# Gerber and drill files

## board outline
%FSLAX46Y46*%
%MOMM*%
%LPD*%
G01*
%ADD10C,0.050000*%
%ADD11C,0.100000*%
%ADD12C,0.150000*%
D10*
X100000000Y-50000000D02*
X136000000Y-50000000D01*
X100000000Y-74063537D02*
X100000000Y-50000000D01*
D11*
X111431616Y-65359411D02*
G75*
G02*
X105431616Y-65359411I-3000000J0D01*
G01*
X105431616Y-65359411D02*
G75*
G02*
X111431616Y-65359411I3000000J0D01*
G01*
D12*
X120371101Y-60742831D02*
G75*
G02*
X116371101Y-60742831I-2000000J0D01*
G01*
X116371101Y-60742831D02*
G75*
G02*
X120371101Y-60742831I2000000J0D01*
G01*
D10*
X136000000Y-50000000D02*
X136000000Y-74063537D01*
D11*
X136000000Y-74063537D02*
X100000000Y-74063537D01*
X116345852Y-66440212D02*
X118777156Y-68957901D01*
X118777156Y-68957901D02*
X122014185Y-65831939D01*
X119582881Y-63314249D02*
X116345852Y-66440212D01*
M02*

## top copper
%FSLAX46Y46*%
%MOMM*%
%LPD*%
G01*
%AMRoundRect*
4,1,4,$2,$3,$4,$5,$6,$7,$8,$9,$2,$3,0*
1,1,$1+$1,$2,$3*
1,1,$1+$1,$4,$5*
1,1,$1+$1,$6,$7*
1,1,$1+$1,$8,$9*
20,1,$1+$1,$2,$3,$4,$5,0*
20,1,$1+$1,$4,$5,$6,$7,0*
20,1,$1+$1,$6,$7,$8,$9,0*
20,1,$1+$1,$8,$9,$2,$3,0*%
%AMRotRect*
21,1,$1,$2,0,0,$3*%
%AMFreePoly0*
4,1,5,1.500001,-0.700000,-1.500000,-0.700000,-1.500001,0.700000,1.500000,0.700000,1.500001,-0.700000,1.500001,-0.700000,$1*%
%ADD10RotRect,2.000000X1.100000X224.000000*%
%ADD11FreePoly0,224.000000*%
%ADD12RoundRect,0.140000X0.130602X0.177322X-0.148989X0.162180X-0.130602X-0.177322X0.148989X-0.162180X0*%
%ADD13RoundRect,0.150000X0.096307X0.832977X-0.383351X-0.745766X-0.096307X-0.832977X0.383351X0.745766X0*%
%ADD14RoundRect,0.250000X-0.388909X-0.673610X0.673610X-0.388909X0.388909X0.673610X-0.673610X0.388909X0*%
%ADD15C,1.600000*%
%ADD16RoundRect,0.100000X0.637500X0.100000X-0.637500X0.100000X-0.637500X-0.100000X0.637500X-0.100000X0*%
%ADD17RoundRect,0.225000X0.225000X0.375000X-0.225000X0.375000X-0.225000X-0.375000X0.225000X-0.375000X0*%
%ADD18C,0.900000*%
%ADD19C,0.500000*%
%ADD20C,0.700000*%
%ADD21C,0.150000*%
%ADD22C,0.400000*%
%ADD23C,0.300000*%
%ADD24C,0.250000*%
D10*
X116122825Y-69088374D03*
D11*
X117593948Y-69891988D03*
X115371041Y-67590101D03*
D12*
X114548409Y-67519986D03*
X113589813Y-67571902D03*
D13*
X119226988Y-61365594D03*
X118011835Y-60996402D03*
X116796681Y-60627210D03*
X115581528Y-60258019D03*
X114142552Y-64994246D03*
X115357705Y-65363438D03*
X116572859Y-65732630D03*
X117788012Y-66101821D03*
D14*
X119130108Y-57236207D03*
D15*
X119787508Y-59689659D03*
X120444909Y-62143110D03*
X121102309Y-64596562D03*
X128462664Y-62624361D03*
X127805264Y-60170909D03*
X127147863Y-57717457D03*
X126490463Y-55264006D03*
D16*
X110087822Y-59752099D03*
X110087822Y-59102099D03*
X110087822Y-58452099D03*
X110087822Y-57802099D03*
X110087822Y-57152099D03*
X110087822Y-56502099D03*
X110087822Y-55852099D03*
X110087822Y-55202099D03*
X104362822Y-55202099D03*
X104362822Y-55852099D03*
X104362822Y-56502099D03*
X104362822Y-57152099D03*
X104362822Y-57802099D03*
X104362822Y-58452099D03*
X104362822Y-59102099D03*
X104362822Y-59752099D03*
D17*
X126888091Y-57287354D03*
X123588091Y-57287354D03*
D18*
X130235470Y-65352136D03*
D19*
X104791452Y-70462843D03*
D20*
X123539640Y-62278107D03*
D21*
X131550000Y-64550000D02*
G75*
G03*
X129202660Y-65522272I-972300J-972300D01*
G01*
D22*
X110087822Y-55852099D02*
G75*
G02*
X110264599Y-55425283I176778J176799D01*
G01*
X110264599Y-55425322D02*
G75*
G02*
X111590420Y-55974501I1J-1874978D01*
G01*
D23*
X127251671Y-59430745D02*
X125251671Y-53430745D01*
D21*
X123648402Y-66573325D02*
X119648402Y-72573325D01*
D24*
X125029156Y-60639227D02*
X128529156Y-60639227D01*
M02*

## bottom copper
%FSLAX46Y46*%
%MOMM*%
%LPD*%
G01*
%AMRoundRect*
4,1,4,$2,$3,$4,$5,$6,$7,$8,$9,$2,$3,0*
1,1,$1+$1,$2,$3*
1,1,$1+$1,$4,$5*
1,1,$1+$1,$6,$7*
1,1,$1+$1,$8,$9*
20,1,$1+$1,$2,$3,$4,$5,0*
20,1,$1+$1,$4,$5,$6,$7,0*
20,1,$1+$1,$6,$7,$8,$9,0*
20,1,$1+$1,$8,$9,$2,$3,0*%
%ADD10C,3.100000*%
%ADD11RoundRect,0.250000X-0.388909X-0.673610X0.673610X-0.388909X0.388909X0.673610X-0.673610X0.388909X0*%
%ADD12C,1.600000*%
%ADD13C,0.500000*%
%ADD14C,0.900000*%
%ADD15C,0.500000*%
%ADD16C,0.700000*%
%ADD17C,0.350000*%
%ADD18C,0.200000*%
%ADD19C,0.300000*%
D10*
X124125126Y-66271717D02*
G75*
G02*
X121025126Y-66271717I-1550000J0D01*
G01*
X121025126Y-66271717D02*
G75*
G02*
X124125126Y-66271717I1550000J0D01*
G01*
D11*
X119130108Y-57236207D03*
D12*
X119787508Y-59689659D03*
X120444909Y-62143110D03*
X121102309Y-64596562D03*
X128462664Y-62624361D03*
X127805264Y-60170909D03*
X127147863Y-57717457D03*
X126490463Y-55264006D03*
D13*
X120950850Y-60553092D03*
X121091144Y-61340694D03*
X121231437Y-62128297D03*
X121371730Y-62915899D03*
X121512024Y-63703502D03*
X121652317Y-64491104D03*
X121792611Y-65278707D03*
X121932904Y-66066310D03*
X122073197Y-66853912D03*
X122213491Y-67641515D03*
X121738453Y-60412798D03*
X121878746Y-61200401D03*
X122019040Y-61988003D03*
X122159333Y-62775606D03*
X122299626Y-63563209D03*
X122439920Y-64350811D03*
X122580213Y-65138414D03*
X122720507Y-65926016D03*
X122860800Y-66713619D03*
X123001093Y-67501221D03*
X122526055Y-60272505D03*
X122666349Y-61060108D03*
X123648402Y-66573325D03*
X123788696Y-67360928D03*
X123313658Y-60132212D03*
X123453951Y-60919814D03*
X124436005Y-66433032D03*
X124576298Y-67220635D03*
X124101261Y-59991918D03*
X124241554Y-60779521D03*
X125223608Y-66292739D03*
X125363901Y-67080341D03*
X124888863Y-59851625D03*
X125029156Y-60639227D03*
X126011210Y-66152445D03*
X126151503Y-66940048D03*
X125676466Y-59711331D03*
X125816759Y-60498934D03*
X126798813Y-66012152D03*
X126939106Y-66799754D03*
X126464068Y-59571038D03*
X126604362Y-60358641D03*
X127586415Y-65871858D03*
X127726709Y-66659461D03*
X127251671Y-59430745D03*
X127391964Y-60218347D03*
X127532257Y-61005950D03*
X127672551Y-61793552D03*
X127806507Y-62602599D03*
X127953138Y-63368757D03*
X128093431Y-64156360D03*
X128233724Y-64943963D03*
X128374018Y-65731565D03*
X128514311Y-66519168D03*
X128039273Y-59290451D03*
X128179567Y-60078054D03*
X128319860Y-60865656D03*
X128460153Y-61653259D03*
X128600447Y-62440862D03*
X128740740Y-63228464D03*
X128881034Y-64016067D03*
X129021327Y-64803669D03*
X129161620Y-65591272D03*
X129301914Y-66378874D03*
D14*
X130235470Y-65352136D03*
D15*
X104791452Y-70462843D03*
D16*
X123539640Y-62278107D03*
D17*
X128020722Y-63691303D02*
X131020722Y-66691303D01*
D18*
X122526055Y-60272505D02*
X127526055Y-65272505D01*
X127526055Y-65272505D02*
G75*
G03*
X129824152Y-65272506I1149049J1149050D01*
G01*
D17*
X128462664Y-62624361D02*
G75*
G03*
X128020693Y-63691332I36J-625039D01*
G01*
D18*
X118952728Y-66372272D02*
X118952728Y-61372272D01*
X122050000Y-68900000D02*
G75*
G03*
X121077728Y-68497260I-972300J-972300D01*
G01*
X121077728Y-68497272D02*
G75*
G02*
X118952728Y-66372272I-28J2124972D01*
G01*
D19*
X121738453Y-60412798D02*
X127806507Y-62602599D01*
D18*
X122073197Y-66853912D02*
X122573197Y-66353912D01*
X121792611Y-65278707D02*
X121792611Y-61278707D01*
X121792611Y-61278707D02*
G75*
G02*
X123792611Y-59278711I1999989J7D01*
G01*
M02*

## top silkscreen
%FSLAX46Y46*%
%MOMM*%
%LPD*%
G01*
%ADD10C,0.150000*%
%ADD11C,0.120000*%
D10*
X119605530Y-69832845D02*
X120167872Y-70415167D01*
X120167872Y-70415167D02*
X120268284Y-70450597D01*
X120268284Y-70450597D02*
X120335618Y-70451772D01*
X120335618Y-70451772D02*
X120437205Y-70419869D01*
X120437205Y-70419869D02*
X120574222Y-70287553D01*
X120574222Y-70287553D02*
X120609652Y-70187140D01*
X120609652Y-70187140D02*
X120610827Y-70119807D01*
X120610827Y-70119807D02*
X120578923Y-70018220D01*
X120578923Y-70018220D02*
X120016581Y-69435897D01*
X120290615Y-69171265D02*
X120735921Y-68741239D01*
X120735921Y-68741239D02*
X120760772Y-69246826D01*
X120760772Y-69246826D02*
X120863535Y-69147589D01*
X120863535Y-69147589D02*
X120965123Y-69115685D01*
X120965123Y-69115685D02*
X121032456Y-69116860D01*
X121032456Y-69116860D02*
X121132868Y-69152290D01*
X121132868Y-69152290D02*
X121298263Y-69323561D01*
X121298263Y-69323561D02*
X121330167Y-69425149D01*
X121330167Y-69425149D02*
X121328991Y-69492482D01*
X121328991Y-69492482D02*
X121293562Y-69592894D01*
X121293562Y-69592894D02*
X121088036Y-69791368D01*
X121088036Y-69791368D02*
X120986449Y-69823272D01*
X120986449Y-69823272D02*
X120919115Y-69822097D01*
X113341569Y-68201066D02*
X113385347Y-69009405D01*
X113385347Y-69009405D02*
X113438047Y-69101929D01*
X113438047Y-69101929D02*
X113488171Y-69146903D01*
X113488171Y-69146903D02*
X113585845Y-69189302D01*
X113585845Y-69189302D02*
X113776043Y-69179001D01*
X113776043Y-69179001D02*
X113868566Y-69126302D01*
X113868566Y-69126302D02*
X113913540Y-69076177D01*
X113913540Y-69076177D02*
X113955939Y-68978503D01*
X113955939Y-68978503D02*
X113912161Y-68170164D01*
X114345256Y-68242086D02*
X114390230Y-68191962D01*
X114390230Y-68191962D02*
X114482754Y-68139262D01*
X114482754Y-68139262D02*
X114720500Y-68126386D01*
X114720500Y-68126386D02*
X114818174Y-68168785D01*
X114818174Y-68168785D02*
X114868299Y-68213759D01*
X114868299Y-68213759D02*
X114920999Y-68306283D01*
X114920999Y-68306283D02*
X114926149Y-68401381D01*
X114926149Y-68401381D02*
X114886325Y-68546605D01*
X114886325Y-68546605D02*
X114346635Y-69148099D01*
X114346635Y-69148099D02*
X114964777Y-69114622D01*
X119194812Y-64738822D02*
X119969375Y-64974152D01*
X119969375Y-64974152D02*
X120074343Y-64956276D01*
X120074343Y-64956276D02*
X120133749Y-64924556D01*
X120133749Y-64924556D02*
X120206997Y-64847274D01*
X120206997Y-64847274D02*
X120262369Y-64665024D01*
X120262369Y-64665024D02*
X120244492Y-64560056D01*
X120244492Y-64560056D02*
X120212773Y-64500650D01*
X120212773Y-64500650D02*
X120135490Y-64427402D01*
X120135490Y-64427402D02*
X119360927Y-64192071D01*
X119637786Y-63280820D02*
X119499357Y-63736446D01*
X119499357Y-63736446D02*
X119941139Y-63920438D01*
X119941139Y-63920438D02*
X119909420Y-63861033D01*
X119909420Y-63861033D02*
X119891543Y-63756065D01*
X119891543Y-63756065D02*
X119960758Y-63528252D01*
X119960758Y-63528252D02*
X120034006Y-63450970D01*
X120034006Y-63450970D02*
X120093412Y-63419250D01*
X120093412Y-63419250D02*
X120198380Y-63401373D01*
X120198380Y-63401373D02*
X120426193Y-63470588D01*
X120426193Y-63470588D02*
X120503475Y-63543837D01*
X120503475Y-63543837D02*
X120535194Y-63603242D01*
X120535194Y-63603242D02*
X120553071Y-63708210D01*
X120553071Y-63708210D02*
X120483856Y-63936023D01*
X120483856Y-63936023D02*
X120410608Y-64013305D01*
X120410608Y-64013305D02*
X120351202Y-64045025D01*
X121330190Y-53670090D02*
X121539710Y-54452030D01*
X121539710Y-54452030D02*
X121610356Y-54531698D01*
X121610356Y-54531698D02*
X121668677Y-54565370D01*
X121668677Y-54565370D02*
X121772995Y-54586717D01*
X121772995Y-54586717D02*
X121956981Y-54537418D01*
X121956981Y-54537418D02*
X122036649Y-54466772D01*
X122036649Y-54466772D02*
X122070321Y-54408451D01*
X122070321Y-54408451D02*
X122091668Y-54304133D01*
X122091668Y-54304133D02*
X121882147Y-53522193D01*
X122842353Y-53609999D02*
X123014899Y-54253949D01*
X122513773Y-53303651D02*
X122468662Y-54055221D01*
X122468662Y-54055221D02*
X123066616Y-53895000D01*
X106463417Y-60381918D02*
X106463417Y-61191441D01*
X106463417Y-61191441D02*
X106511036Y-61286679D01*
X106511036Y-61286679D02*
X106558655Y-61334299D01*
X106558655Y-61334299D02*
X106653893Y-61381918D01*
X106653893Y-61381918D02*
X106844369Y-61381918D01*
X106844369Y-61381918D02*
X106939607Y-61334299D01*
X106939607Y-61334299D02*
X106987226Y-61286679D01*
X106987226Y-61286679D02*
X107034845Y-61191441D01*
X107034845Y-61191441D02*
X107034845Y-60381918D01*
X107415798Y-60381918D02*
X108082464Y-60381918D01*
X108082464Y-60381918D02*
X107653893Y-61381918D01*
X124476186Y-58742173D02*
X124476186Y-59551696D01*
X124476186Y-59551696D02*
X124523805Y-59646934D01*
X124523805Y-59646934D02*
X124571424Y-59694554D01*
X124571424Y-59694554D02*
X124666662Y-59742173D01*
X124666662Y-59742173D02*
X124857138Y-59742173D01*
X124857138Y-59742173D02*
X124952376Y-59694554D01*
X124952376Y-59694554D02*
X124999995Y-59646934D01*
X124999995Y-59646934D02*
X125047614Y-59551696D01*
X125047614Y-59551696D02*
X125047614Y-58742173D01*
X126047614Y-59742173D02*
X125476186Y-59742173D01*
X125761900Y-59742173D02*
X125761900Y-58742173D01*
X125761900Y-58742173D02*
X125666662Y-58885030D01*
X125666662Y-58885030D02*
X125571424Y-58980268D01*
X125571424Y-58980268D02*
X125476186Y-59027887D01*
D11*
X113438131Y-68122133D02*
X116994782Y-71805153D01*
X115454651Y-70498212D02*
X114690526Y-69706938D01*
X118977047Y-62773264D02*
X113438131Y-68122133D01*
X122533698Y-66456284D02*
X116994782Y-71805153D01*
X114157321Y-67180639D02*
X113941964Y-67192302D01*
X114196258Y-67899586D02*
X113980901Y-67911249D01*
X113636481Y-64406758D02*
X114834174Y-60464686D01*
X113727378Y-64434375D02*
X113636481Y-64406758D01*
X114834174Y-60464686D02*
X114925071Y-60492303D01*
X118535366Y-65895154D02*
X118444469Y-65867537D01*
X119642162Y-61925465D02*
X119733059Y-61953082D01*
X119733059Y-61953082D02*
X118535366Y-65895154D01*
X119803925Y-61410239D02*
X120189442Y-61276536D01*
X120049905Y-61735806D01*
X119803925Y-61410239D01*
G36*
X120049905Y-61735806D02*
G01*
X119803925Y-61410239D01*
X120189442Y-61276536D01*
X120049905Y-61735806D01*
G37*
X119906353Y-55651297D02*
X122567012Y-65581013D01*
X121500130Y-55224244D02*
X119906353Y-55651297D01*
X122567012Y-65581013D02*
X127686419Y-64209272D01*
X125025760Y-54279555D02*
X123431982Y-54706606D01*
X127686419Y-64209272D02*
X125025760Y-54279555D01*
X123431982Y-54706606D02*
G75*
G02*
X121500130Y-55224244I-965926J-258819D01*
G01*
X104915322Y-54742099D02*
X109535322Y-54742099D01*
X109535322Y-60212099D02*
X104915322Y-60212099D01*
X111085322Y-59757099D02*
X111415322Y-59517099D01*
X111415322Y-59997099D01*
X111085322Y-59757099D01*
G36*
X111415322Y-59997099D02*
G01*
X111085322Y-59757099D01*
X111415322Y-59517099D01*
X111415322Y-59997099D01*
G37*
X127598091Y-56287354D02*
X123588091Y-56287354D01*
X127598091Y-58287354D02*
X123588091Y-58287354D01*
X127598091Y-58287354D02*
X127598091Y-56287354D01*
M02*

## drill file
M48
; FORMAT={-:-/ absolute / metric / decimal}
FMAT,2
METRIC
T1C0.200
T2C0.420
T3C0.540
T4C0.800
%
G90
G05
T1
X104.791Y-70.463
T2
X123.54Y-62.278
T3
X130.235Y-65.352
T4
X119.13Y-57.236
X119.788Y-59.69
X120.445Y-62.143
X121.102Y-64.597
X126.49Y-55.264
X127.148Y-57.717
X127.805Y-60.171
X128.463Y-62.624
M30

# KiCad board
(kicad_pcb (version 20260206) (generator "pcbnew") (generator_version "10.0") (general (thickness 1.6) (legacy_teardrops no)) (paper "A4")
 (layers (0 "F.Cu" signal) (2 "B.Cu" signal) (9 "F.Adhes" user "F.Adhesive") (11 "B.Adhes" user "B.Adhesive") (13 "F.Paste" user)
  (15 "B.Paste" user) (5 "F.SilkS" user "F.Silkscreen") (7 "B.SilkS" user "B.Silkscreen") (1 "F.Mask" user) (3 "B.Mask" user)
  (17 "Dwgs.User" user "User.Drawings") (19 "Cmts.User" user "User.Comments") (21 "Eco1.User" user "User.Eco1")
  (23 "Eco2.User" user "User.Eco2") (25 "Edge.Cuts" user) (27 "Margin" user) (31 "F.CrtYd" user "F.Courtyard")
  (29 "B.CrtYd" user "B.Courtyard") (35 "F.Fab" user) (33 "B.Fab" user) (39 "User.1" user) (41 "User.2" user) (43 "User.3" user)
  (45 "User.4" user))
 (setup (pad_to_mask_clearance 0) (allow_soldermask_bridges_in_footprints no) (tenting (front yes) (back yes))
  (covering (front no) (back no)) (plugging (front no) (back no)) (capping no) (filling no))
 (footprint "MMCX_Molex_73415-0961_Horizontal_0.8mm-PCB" (layer "F.Cu") (at 118.101009 67.178063 -136)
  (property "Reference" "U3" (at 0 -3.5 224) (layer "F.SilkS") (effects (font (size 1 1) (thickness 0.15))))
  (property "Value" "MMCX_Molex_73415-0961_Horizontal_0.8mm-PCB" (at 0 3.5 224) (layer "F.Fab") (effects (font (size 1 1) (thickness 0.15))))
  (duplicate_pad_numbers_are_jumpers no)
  (fp_line (start 4.01 2.56) (end 4.01 -2.56) (stroke (width 0.12) (type solid)) (layer "F.SilkS"))
  (fp_line (start 4.21 -0.550001) (end 4.21 0.55) (stroke (width 0.12) (type solid)) (layer "F.SilkS"))
  (fp_line (start -3.689999 2.56) (end 4.01 2.56) (stroke (width 0.12) (type solid)) (layer "F.SilkS"))
  (fp_line (start -3.689999 -2.56) (end 4.01 -2.56) (stroke (width 0.12) (type solid)) (layer "F.SilkS"))
  (fp_line (start 0.75 1.75) (end 0.75 -1.749999) (stroke (width 0.1) (type solid)) (layer "Edge.Cuts"))
  (fp_line (start 0.75 -1.749999) (end -3.75 -1.75) (stroke (width 0.1) (type solid)) (layer "Edge.Cuts"))
  (fp_line (start -3.75 1.75) (end 0.75 1.75) (stroke (width 0.1) (type solid)) (layer "Edge.Cuts"))
  (pad "1" smd rect (at 2.75 -0.000001 224) (size 2 1.1) (layers "F.Cu" "F.Mask" "F.Paste") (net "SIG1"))
  (pad "2" smd custom (at 2.25 -1.6 224) (size 3 1.4) (layers "F.Cu" "F.Mask" "F.Paste") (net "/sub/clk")
   (options (clearance outline) (anchor rect)) (primitives))
  (pad "2" smd custom (at 2.25 1.6 224) (size 3 1.4) (layers "F.Cu" "F.Mask" "F.Paste") (options (clearance outline) (anchor rect))
   (primitives)))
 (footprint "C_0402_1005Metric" (layer "F.Cu") (at 114.069111 67.545944 -176.9)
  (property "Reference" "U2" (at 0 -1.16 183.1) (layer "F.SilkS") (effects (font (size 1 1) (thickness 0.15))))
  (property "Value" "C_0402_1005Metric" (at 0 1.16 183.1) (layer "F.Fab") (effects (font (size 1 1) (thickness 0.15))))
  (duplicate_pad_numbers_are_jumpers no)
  (fp_line (start -0.107836 0.36) (end 0.107836 0.36) (stroke (width 0.12) (type solid)) (layer "F.SilkS"))
  (fp_line (start -0.107836 -0.36) (end 0.107836 -0.36) (stroke (width 0.12) (type solid)) (layer "F.SilkS"))
  (pad "1" smd roundrect (at -0.48 0 183.1) (size 0.56 0.62) (layers "F.Cu" "F.Mask" "F.Paste") (roundrect_rratio 0.25))
  (pad "2" smd roundrect (at 0.48 0 183.1) (size 0.56 0.62) (layers "F.Cu" "F.Mask" "F.Paste") (roundrect_rratio 0.25) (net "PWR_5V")))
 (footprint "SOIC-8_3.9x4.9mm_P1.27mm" (layer "F.Cu") (at 116.68477 63.17992 -106.9)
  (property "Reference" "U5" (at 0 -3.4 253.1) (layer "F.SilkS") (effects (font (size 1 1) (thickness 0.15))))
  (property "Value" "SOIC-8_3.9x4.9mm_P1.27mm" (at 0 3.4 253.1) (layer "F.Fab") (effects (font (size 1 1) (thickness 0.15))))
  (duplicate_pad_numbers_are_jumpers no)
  (fp_line (start 2.06 2.56) (end -2.06 2.56) (stroke (width 0.12) (type solid)) (layer "F.SilkS"))
  (fp_line (start 2.06 2.465) (end 2.06 2.56) (stroke (width 0.12) (type solid)) (layer "F.SilkS"))
  (fp_line (start -2.06 2.56) (end -2.06 2.465) (stroke (width 0.12) (type solid)) (layer "F.SilkS"))
  (fp_line (start 2.06 -2.56) (end 2.06 -2.465) (stroke (width 0.12) (type solid)) (layer "F.SilkS"))
  (fp_line (start -2.06 -2.465) (end -2.06 -2.56) (stroke (width 0.12) (type solid)) (layer "F.SilkS"))
  (fp_line (start -2.06 -2.56) (end 2.06 -2.56) (stroke (width 0.12) (type solid)) (layer "F.SilkS"))
  (fp_poly (pts (xy -2.6 -2.47) (xy -2.84 -2.8) (xy -2.36 -2.8)) (stroke (width 0.12) (type solid)) (fill yes) (layer "F.SilkS"))
  (pad "1" smd roundrect (at -2.475 -1.905 253.1) (size 1.95 0.6) (layers "F.Cu" "F.Mask" "F.Paste") (roundrect_rratio 0.25) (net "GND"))
  (pad "2" smd roundrect (at -2.475 -0.635 253.1) (size 1.95 0.6) (layers "F.Cu" "F.Mask" "F.Paste") (roundrect_rratio 0.25) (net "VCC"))
  (pad "3" smd roundrect (at -2.475 0.635 253.1) (size 1.95 0.6) (layers "F.Cu" "F.Mask" "F.Paste") (roundrect_rratio 0.25))
  (pad "4" smd roundrect (at -2.475 1.905 253.1) (size 1.95 0.6) (layers "F.Cu" "F.Mask" "F.Paste") (roundrect_rratio 0.25) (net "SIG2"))
  (pad "5" smd roundrect (at 2.475 1.905 253.1) (size 1.95 0.6) (layers "F.Cu" "F.Mask" "F.Paste") (roundrect_rratio 0.25) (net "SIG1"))
  (pad "6" smd roundrect (at 2.475 0.635 253.1) (size 1.95 0.6) (layers "F.Cu" "F.Mask" "F.Paste") (roundrect_rratio 0.25))
  (pad "7" smd roundrect (at 2.475 -0.635 253.1) (size 1.95 0.6) (layers "F.Cu" "F.Mask" "F.Paste") (roundrect_rratio 0.25) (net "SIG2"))
  (pad "8" smd roundrect (at 2.475 -1.905 253.1) (size 1.95 0.6) (layers "F.Cu" "F.Mask" "F.Paste") (roundrect_rratio 0.25) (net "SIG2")))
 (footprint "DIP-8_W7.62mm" (layer "F.Cu") (at 119.130108 57.236207 15)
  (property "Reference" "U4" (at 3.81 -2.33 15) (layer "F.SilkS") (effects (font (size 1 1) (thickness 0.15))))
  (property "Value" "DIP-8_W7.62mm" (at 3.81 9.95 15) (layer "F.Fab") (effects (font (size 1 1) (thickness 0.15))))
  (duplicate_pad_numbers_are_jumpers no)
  (fp_line (start 1.16 -1.329999) (end 1.16 8.95) (stroke (width 0.12) (type solid)) (layer "F.SilkS"))
  (fp_line (start 2.81 -1.33) (end 1.16 -1.329999) (stroke (width 0.12) (type solid)) (layer "F.SilkS"))
  (fp_line (start 1.16 8.95) (end 6.46 8.95) (stroke (width 0.12) (type solid)) (layer "F.SilkS"))
  (fp_line (start 6.46 -1.33) (end 4.81 -1.33) (stroke (width 0.12) (type solid)) (layer "F.SilkS"))
  (fp_line (start 6.46 8.95) (end 6.46 -1.33) (stroke (width 0.12) (type solid)) (layer "F.SilkS"))
  (fp_arc (start 4.81 -1.33) (mid 3.81 -0.33) (end 2.81 -1.33) (stroke (width 0.12) (type solid)) (layer "F.SilkS"))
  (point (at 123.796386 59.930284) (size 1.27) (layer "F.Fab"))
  (pad "1" thru_hole roundrect (at 0 0 15) (size 1.6 1.6) (drill 0.8) (layers "*.Cu" "*.Mask") (remove_unused_layers no)
   (roundrect_rratio 0.15625) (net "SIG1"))
  (pad "2" thru_hole circle (at 0 2.54 15) (size 1.6 1.6) (drill 0.8) (layers "*.Cu" "*.Mask") (remove_unused_layers no) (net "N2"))
  (pad "3" thru_hole circle (at 0 5.08 15) (size 1.6 1.6) (drill 0.8) (layers "*.Cu" "*.Mask") (remove_unused_layers no) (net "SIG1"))
  (pad "4" thru_hole circle (at 0 7.62 15) (size 1.6 1.6) (drill 0.8) (layers "*.Cu" "*.Mask") (remove_unused_layers no))
  (pad "5" thru_hole circle (at 7.62 7.62 15) (size 1.6 1.6) (drill 0.8) (layers "*.Cu" "*.Mask") (remove_unused_layers no) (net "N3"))
  (pad "6" thru_hole circle (at 7.62 5.08 15) (size 1.6 1.6) (drill 0.8) (layers "*.Cu" "*.Mask") (remove_unused_layers no) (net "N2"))
  (pad "7" thru_hole circle (at 7.62 2.539999 15) (size 1.6 1.6) (drill 0.8) (layers "*.Cu" "*.Mask") (remove_unused_layers no) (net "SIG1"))
  (pad "8" thru_hole circle (at 7.62 0 15) (size 1.6 1.6) (drill 0.8) (layers "*.Cu" "*.Mask") (remove_unused_layers no) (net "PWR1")))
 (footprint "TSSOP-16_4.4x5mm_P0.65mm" (layer "F.Cu") (at 107.225322 57.477099 180)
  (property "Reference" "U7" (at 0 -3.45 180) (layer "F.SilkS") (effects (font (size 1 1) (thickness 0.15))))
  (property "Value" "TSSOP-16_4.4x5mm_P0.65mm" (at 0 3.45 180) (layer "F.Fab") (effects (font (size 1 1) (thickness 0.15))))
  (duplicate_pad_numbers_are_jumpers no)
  (fp_line (start 2.31 2.735) (end -2.31 2.735) (stroke (width 0.12) (type solid)) (layer "F.SilkS"))
  (fp_line (start -2.31 -2.735) (end 2.31 -2.735) (stroke (width 0.12) (type solid)) (layer "F.SilkS"))
  (fp_poly (pts (xy -3.86 -2.28) (xy -4.19 -2.04) (xy -4.19 -2.52)) (stroke (width 0.12) (type solid)) (fill yes) (layer "F.SilkS"))
  (pad "1" smd roundrect (at -2.8625 -2.275 180) (size 1.475 0.4) (layers "F.Cu" "F.Mask" "F.Paste") (roundrect_rratio 0.25) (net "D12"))
  (pad "2" smd roundrect (at -2.8625 -1.625 180) (size 1.475 0.4) (layers "F.Cu" "F.Mask" "F.Paste") (roundrect_rratio 0.25) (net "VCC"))
  (pad "3" smd roundrect (at -2.8625 -0.975 180) (size 1.475 0.4) (layers "F.Cu" "F.Mask" "F.Paste") (roundrect_rratio 0.25) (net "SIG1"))
  (pad "4" smd roundrect (at -2.8625 -0.325 180) (size 1.475 0.4) (layers "F.Cu" "F.Mask" "F.Paste") (roundrect_rratio 0.25) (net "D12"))
  (pad "5" smd roundrect (at -2.8625 0.325 180) (size 1.475 0.4) (layers "F.Cu" "F.Mask" "F.Paste") (roundrect_rratio 0.25))
  (pad "6" smd roundrect (at -2.8625 0.975 180) (size 1.475 0.4) (layers "F.Cu" "F.Mask" "F.Paste") (roundrect_rratio 0.25))
  (pad "7" smd roundrect (at -2.8625 1.625 180) (size 1.475 0.4) (layers "F.Cu" "F.Mask" "F.Paste") (roundrect_rratio 0.25) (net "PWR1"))
  (pad "8" smd roundrect (at -2.8625 2.275 180) (size 1.475 0.4) (layers "F.Cu" "F.Mask" "F.Paste") (roundrect_rratio 0.25))
  (pad "9" smd roundrect (at 2.8625 2.275 180) (size 1.475 0.4) (layers "F.Cu" "F.Mask" "F.Paste") (roundrect_rratio 0.25) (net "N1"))
  (pad "10" smd roundrect (at 2.8625 1.625 180) (size 1.475 0.4) (layers "F.Cu" "F.Mask" "F.Paste") (roundrect_rratio 0.25) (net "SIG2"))
  (pad "11" smd roundrect (at 2.8625 0.975 180) (size 1.475 0.4) (layers "F.Cu" "F.Mask" "F.Paste") (roundrect_rratio 0.25) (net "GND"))
  (pad "12" smd roundrect (at 2.8625 0.325 180) (size 1.475 0.4) (layers "F.Cu" "F.Mask" "F.Paste") (roundrect_rratio 0.25))
  (pad "13" smd roundrect (at 2.8625 -0.325 180) (size 1.475 0.4) (layers "F.Cu" "F.Mask" "F.Paste") (roundrect_rratio 0.25)
   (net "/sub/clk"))
  (pad "14" smd roundrect (at 2.8625 -0.975 180) (size 1.475 0.4) (layers "F.Cu" "F.Mask" "F.Paste") (roundrect_rratio 0.25) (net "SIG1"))
  (pad "15" smd roundrect (at 2.8625 -1.625 180) (size 1.475 0.4) (layers "F.Cu" "F.Mask" "F.Paste") (roundrect_rratio 0.25) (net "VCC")
   (clearance 0.1))
  (pad "16" smd roundrect (at 2.8625 -2.275 180) (size 1.475 0.4) (layers "F.Cu" "F.Mask" "F.Paste") (roundrect_rratio 0.25) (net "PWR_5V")))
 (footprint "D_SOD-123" (layer "F.Cu") (at 125.238091 57.287354 180)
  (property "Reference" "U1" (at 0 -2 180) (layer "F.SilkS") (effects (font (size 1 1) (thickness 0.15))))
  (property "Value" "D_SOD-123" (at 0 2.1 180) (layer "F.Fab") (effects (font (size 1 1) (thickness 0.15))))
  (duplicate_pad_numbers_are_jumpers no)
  (fp_line (start -2.36 1) (end 1.65 1) (stroke (width 0.12) (type solid)) (layer "F.SilkS"))
  (fp_line (start -2.36 -1) (end 1.65 -1) (stroke (width 0.12) (type solid)) (layer "F.SilkS"))
  (fp_line (start -2.36 -1) (end -2.36 1) (stroke (width 0.12) (type solid)) (layer "F.SilkS"))
  (pad "1" smd roundrect (at -1.65 0 180) (size 0.9 1.2) (layers "F.Cu" "F.Mask" "F.Paste") (roundrect_rratio 0.25) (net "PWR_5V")
   (clearance 0.1))
  (pad "2" smd roundrect (at 1.65 0 180) (size 0.9 1.2) (layers "F.Cu" "F.Mask" "F.Paste") (roundrect_rratio 0.25) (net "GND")
   (clearance 0.35)))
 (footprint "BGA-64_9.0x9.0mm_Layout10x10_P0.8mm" (layer "B.Cu") (at 125.126382 63.465983 -79.9)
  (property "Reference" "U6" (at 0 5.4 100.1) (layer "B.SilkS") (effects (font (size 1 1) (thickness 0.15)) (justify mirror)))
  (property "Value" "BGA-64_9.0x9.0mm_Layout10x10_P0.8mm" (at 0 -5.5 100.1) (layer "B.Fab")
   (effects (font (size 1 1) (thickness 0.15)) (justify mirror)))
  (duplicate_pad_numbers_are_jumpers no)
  (pad "A1" smd circle (at -3.6 3.6 280.1) (size 0.5 0.5) (layers "B.Cu" "B.Mask" "B.Paste") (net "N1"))
  (pad "A2" smd circle (at -2.8 3.6 280.1) (size 0.5 0.5) (layers "B.Cu" "B.Mask" "B.Paste") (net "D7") (clearance 0.1))
  (pad "A3" smd circle (at -2 3.6 280.1) (size 0.5 0.5) (layers "B.Cu" "B.Mask" "B.Paste"))
  (pad "A4" smd circle (at -1.2 3.6 280.1) (size 0.5 0.5) (layers "B.Cu" "B.Mask" "B.Paste") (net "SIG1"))
  (pad "A5" smd circle (at -0.4 3.6 280.1) (size 0.5 0.5) (layers "B.Cu" "B.Mask" "B.Paste") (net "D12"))
  (pad "A6" smd circle (at 0.399999 3.6 280.1) (size 0.5 0.5) (layers "B.Cu" "B.Mask" "B.Paste") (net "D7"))
  (pad "A7" smd circle (at 1.2 3.6 280.1) (size 0.5 0.5) (layers "B.Cu" "B.Mask" "B.Paste") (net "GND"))
  (pad "A8" smd circle (at 2 3.6 280.1) (size 0.5 0.5) (layers "B.Cu" "B.Mask" "B.Paste") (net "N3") (clearance 0.35))
  (pad "A9" smd circle (at 2.8 3.6 280.1) (size 0.5 0.5) (layers "B.Cu" "B.Mask" "B.Paste") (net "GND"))
  (pad "A10" smd circle (at 3.6 3.6 280.1) (size 0.5 0.5) (layers "B.Cu" "B.Mask" "B.Paste") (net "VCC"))
  (pad "B1" smd circle (at -3.6 2.8 280.1) (size 0.5 0.5) (layers "B.Cu" "B.Mask" "B.Paste") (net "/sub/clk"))
  (pad "B2" smd circle (at -2.8 2.8 280.1) (size 0.5 0.5) (layers "B.Cu" "B.Mask" "B.Paste") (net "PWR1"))
  (pad "B3" smd circle (at -2 2.8 280.1) (size 0.5 0.5) (layers "B.Cu" "B.Mask" "B.Paste") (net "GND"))
  (pad "B4" smd circle (at -1.2 2.8 280.1) (size 0.5 0.5) (layers "B.Cu" "B.Mask" "B.Paste") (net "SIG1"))
  (pad "B5" smd circle (at -0.4 2.8 280.1) (size 0.5 0.5) (layers "B.Cu" "B.Mask" "B.Paste") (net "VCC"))
  (pad "B6" smd circle (at 0.4 2.8 280.1) (size 0.5 0.5) (layers "B.Cu" "B.Mask" "B.Paste") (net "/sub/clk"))
  (pad "B7" smd circle (at 1.2 2.8 280.1) (size 0.5 0.5) (layers "B.Cu" "B.Mask" "B.Paste") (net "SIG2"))
  (pad "B8" smd circle (at 2 2.8 280.1) (size 0.5 0.5) (layers "B.Cu" "B.Mask" "B.Paste") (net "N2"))
  (pad "B9" smd circle (at 2.8 2.8 280.1) (size 0.5 0.5) (layers "B.Cu" "B.Mask" "B.Paste") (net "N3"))
  (pad "B10" smd circle (at 3.6 2.8 280.1) (size 0.5 0.5) (layers "B.Cu" "B.Mask" "B.Paste"))
  (pad "C1" smd circle (at -3.6 2 280.1) (size 0.5 0.5) (layers "B.Cu" "B.Mask" "B.Paste"))
  (pad "C2" smd circle (at -2.8 2 280.1) (size 0.5 0.5) (layers "B.Cu" "B.Mask" "B.Paste"))
  (pad "C9" smd circle (at 2.8 2 280.1) (size 0.5 0.5) (layers "B.Cu" "B.Mask" "B.Paste") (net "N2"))
  (pad "C10" smd circle (at 3.6 2 280.1) (size 0.5 0.5) (layers "B.Cu" "B.Mask" "B.Paste"))
  (pad "D1" smd circle (at -3.6 1.2 280.1) (size 0.5 0.5) (layers "B.Cu" "B.Mask" "B.Paste"))
  (pad "D2" smd circle (at -2.8 1.2 280.1) (size 0.5 0.5) (layers "B.Cu" "B.Mask" "B.Paste") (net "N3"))
  (pad "D9" smd circle (at 2.8 1.2 280.1) (size 0.5 0.5) (layers "B.Cu" "B.Mask" "B.Paste") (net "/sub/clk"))
  (pad "D10" smd circle (at 3.6 1.2 280.1) (size 0.5 0.5) (layers "B.Cu" "B.Mask" "B.Paste") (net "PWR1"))
  (pad "E1" smd circle (at -3.6 0.399999 280.1) (size 0.5 0.5) (layers "B.Cu" "B.Mask" "B.Paste") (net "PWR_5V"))
  (pad "E2" smd circle (at -2.8 0.4 280.1) (size 0.5 0.5) (layers "B.Cu" "B.Mask" "B.Paste") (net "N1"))
  (pad "E9" smd circle (at 2.8 0.4 280.1) (size 0.5 0.5) (layers "B.Cu" "B.Mask" "B.Paste") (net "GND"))
  (pad "E10" smd circle (at 3.6 0.4 280.1) (size 0.5 0.5) (layers "B.Cu" "B.Mask" "B.Paste"))
  (pad "F1" smd circle (at -3.6 -0.4 280.1) (size 0.5 0.5) (layers "B.Cu" "B.Mask" "B.Paste") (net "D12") (clearance 0.35))
  (pad "F2" smd circle (at -2.8 -0.4 280.1) (size 0.5 0.5) (layers "B.Cu" "B.Mask" "B.Paste"))
  (pad "F9" smd circle (at 2.8 -0.4 280.1) (size 0.5 0.5) (layers "B.Cu" "B.Mask" "B.Paste") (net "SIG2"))
  (pad "F10" smd circle (at 3.6 -0.399999 280.1) (size 0.5 0.5) (layers "B.Cu" "B.Mask" "B.Paste") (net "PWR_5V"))
  (pad "G1" smd circle (at -3.6 -1.2 280.1) (size 0.5 0.5) (layers "B.Cu" "B.Mask" "B.Paste") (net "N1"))
  (pad "G2" smd circle (at -2.8 -1.2 280.1) (size 0.5 0.5) (layers "B.Cu" "B.Mask" "B.Paste") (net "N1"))
  (pad "G9" smd circle (at 2.8 -1.2 280.1) (size 0.5 0.5) (layers "B.Cu" "B.Mask" "B.Paste") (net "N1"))
  (pad "G10" smd circle (at 3.6 -1.2 280.1) (size 0.5 0.5) (layers "B.Cu" "B.Mask" "B.Paste") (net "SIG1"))
  (pad "H1" smd circle (at -3.6 -2 280.1) (size 0.5 0.5) (layers "B.Cu" "B.Mask" "B.Paste") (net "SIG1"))
  (pad "H2" smd circle (at -2.8 -2 280.1) (size 0.5 0.5) (layers "B.Cu" "B.Mask" "B.Paste") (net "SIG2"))
  (pad "H9" smd circle (at 2.8 -2 280.1) (size 0.5 0.5) (layers "B.Cu" "B.Mask" "B.Paste") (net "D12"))
  (pad "H10" smd circle (at 3.6 -2 280.1) (size 0.5 0.5) (layers "B.Cu" "B.Mask" "B.Paste"))
  (pad "J1" smd circle (at -3.6 -2.8 280.1) (size 0.5 0.5) (layers "B.Cu" "B.Mask" "B.Paste") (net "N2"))
  (pad "J2" smd circle (at -2.8 -2.8 280.1) (size 0.5 0.5) (layers "B.Cu" "B.Mask" "B.Paste") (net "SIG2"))
  (pad "J3" smd circle (at -2 -2.8 280.1) (size 0.5 0.5) (layers "B.Cu" "B.Mask" "B.Paste") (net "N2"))
  (pad "J4" smd circle (at -1.2 -2.8 280.1) (size 0.5 0.5) (layers "B.Cu" "B.Mask" "B.Paste") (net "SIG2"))
  (pad "J5" smd circle (at -0.38 -2.79 280.1) (size 0.5 0.5) (layers "B.Cu" "B.Mask" "B.Paste") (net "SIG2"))
  (pad "J6" smd circle (at 0.4 -2.8 280.1) (size 0.5 0.5) (layers "B.Cu" "B.Mask" "B.Paste") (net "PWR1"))
  (pad "J7" smd circle (at 1.2 -2.8 280.1) (size 0.5 0.5) (layers "B.Cu" "B.Mask" "B.Paste") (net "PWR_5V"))
  (pad "J8" smd circle (at 2 -2.8 280.1) (size 0.5 0.5) (layers "B.Cu" "B.Mask" "B.Paste"))
  (pad "J9" smd circle (at 2.8 -2.8 280.1) (size 0.5 0.5) (layers "B.Cu" "B.Mask" "B.Paste"))
  (pad "J10" smd circle (at 3.6 -2.8 280.1) (size 0.5 0.5) (layers "B.Cu" "B.Mask" "B.Paste"))
  (pad "K1" smd circle (at -3.6 -3.6 280.1) (size 0.5 0.5) (layers "B.Cu" "B.Mask" "B.Paste") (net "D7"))
  (pad "K2" smd circle (at -2.8 -3.6 280.1) (size 0.5 0.5) (layers "B.Cu" "B.Mask" "B.Paste") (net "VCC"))
  (pad "K3" smd circle (at -2 -3.6 280.1) (size 0.5 0.5) (layers "B.Cu" "B.Mask" "B.Paste"))
  (pad "K4" smd circle (at -1.2 -3.6 280.1) (size 0.5 0.5) (layers "B.Cu" "B.Mask" "B.Paste") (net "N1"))
  (pad "K5" smd circle (at -0.399999 -3.6 280.1) (size 0.5 0.5) (layers "B.Cu" "B.Mask" "B.Paste") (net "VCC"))
  (pad "K6" smd circle (at 0.4 -3.6 280.1) (size 0.5 0.5) (layers "B.Cu" "B.Mask" "B.Paste") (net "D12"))
  (pad "K7" smd circle (at 1.2 -3.6 280.1) (size 0.5 0.5) (layers "B.Cu" "B.Mask" "B.Paste") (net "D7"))
  (pad "K8" smd circle (at 2 -3.6 280.1) (size 0.5 0.5) (layers "B.Cu" "B.Mask" "B.Paste"))
  (pad "K9" smd circle (at 2.8 -3.6 280.1) (size 0.5 0.5) (layers "B.Cu" "B.Mask" "B.Paste"))
  (pad "K10" smd circle (at 3.6 -3.6 280.1) (size 0.5 0.5) (layers "B.Cu" "B.Mask" "B.Paste")))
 (gr_circle (center 122.575126 66.271717) (end 125.575126 66.271717) (stroke (width 0.2) (type default)) (fill yes) (layer "B.Cu"))
 (gr_line (start 100 50) (end 136 50) (stroke (width 0.05) (type default)) (layer "Edge.Cuts"))
 (gr_line (start 100 74.063537) (end 100 50) (stroke (width 0.05) (type default)) (layer "Edge.Cuts"))
 (gr_circle (center 108.431616 65.359411) (end 111.431616 65.359411) (stroke (width 0.1) (type default)) (fill no) (layer "Edge.Cuts"))
 (gr_circle (center 118.371101 60.742831) (end 120.371101 60.742831) (stroke (width 0.15) (type default)) (fill no) (layer "Edge.Cuts"))
 (gr_line (start 136 50) (end 136 74.063537) (stroke (width 0.05) (type default)) (layer "Edge.Cuts"))
 (gr_line (start 136 74.063537) (end 100 74.063537) (stroke (width 0.1) (type default)) (layer "Edge.Cuts"))
 (arc (start 131.55 64.55) (mid 130.051538 64.251937) (end 129.202728 65.522272) (width 0.15) (layer "F.Cu") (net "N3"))
 (segment (start 128.020722 63.691303) (end 131.020722 66.691303) (width 0.35) (layer "B.Cu") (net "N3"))
 (segment (start 122.526055 60.272505) (end 127.526055 65.272505) (width 0.2) (locked yes) (layer "B.Cu") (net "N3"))
 (arc (start 127.526055 65.272505) (mid 128.675104 65.748456) (end 129.824152 65.272505) (width 0.2) (layer "B.Cu") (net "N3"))
 (arc (start 128.462664 62.624361) (mid 127.885239 63.010184) (end 128.020722 63.691303) (width 0.35) (layer "B.Cu") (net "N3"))
 (via (at 130.23547 65.352136) (size 0.9) (drill 0.54) (layers "F.Cu" "B.Cu") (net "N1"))
 (segment (start 118.952728 66.372272) (end 118.952728 61.372272) (width 0.2) (layer "B.Cu") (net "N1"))
 (arc (start 122.05 68.9) (mid 121.603918 68.601937) (end 121.077728 68.497272) (width 0.2) (layer "B.Cu") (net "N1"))
 (arc (start 121.077728 68.497272) (mid 119.575126 67.874874) (end 118.952728 66.372272) (width 0.2) (layer "B.Cu") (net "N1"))
 (arc (start 110.087822 55.852099) (mid 110.033629 55.579651) (end 110.264599 55.425322) (width 0.4) (layer "F.Cu") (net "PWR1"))
 (arc (start 110.264599 55.425322) (mid 110.98213 55.568048) (end 111.590424 55.974497) (width 0.4) (layer "F.Cu") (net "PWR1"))
 (segment (start 121.738453 60.412798) (end 127.806507 62.602599) (width 0.3) (layer "B.Cu") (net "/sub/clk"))
 (segment (start 127.251671 59.430745) (end 125.251671 53.430745) (width 0.3) (layer "F.Cu") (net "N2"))
 (segment (start 123.648402 66.573325) (end 119.648402 72.573325) (width 0.15) (layer "F.Cu") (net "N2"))
 (via (at 104.791452 70.462843) (size 0.5) (drill 0.2) (layers "F.Cu" "B.Cu") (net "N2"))
 (segment (start 125.029156 60.639227) (end 128.529156 60.639227) (width 0.25) (layer "F.Cu") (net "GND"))
 (via (at 123.53964 62.278107) (size 0.7) (drill 0.42) (layers "F.Cu" "B.Cu") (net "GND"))
 (segment (start 122.073197 66.853912) (end 122.573197 66.353912) (width 0.2) (layer "B.Cu") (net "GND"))
 (segment (start 121.792611 65.278707) (end 121.792611 61.278707) (width 0.2) (layer "B.Cu") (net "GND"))
 (arc (start 121.792611 61.278707) (mid 122.378397 59.864493) (end 123.792611 59.278707) (width 0.2) (layer "B.Cu") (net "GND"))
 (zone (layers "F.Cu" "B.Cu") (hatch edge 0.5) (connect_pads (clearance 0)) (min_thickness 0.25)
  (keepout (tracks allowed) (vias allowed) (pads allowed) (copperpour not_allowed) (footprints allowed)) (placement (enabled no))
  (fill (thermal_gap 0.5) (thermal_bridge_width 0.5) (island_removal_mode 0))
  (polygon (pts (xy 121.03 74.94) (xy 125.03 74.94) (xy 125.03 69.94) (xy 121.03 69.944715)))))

